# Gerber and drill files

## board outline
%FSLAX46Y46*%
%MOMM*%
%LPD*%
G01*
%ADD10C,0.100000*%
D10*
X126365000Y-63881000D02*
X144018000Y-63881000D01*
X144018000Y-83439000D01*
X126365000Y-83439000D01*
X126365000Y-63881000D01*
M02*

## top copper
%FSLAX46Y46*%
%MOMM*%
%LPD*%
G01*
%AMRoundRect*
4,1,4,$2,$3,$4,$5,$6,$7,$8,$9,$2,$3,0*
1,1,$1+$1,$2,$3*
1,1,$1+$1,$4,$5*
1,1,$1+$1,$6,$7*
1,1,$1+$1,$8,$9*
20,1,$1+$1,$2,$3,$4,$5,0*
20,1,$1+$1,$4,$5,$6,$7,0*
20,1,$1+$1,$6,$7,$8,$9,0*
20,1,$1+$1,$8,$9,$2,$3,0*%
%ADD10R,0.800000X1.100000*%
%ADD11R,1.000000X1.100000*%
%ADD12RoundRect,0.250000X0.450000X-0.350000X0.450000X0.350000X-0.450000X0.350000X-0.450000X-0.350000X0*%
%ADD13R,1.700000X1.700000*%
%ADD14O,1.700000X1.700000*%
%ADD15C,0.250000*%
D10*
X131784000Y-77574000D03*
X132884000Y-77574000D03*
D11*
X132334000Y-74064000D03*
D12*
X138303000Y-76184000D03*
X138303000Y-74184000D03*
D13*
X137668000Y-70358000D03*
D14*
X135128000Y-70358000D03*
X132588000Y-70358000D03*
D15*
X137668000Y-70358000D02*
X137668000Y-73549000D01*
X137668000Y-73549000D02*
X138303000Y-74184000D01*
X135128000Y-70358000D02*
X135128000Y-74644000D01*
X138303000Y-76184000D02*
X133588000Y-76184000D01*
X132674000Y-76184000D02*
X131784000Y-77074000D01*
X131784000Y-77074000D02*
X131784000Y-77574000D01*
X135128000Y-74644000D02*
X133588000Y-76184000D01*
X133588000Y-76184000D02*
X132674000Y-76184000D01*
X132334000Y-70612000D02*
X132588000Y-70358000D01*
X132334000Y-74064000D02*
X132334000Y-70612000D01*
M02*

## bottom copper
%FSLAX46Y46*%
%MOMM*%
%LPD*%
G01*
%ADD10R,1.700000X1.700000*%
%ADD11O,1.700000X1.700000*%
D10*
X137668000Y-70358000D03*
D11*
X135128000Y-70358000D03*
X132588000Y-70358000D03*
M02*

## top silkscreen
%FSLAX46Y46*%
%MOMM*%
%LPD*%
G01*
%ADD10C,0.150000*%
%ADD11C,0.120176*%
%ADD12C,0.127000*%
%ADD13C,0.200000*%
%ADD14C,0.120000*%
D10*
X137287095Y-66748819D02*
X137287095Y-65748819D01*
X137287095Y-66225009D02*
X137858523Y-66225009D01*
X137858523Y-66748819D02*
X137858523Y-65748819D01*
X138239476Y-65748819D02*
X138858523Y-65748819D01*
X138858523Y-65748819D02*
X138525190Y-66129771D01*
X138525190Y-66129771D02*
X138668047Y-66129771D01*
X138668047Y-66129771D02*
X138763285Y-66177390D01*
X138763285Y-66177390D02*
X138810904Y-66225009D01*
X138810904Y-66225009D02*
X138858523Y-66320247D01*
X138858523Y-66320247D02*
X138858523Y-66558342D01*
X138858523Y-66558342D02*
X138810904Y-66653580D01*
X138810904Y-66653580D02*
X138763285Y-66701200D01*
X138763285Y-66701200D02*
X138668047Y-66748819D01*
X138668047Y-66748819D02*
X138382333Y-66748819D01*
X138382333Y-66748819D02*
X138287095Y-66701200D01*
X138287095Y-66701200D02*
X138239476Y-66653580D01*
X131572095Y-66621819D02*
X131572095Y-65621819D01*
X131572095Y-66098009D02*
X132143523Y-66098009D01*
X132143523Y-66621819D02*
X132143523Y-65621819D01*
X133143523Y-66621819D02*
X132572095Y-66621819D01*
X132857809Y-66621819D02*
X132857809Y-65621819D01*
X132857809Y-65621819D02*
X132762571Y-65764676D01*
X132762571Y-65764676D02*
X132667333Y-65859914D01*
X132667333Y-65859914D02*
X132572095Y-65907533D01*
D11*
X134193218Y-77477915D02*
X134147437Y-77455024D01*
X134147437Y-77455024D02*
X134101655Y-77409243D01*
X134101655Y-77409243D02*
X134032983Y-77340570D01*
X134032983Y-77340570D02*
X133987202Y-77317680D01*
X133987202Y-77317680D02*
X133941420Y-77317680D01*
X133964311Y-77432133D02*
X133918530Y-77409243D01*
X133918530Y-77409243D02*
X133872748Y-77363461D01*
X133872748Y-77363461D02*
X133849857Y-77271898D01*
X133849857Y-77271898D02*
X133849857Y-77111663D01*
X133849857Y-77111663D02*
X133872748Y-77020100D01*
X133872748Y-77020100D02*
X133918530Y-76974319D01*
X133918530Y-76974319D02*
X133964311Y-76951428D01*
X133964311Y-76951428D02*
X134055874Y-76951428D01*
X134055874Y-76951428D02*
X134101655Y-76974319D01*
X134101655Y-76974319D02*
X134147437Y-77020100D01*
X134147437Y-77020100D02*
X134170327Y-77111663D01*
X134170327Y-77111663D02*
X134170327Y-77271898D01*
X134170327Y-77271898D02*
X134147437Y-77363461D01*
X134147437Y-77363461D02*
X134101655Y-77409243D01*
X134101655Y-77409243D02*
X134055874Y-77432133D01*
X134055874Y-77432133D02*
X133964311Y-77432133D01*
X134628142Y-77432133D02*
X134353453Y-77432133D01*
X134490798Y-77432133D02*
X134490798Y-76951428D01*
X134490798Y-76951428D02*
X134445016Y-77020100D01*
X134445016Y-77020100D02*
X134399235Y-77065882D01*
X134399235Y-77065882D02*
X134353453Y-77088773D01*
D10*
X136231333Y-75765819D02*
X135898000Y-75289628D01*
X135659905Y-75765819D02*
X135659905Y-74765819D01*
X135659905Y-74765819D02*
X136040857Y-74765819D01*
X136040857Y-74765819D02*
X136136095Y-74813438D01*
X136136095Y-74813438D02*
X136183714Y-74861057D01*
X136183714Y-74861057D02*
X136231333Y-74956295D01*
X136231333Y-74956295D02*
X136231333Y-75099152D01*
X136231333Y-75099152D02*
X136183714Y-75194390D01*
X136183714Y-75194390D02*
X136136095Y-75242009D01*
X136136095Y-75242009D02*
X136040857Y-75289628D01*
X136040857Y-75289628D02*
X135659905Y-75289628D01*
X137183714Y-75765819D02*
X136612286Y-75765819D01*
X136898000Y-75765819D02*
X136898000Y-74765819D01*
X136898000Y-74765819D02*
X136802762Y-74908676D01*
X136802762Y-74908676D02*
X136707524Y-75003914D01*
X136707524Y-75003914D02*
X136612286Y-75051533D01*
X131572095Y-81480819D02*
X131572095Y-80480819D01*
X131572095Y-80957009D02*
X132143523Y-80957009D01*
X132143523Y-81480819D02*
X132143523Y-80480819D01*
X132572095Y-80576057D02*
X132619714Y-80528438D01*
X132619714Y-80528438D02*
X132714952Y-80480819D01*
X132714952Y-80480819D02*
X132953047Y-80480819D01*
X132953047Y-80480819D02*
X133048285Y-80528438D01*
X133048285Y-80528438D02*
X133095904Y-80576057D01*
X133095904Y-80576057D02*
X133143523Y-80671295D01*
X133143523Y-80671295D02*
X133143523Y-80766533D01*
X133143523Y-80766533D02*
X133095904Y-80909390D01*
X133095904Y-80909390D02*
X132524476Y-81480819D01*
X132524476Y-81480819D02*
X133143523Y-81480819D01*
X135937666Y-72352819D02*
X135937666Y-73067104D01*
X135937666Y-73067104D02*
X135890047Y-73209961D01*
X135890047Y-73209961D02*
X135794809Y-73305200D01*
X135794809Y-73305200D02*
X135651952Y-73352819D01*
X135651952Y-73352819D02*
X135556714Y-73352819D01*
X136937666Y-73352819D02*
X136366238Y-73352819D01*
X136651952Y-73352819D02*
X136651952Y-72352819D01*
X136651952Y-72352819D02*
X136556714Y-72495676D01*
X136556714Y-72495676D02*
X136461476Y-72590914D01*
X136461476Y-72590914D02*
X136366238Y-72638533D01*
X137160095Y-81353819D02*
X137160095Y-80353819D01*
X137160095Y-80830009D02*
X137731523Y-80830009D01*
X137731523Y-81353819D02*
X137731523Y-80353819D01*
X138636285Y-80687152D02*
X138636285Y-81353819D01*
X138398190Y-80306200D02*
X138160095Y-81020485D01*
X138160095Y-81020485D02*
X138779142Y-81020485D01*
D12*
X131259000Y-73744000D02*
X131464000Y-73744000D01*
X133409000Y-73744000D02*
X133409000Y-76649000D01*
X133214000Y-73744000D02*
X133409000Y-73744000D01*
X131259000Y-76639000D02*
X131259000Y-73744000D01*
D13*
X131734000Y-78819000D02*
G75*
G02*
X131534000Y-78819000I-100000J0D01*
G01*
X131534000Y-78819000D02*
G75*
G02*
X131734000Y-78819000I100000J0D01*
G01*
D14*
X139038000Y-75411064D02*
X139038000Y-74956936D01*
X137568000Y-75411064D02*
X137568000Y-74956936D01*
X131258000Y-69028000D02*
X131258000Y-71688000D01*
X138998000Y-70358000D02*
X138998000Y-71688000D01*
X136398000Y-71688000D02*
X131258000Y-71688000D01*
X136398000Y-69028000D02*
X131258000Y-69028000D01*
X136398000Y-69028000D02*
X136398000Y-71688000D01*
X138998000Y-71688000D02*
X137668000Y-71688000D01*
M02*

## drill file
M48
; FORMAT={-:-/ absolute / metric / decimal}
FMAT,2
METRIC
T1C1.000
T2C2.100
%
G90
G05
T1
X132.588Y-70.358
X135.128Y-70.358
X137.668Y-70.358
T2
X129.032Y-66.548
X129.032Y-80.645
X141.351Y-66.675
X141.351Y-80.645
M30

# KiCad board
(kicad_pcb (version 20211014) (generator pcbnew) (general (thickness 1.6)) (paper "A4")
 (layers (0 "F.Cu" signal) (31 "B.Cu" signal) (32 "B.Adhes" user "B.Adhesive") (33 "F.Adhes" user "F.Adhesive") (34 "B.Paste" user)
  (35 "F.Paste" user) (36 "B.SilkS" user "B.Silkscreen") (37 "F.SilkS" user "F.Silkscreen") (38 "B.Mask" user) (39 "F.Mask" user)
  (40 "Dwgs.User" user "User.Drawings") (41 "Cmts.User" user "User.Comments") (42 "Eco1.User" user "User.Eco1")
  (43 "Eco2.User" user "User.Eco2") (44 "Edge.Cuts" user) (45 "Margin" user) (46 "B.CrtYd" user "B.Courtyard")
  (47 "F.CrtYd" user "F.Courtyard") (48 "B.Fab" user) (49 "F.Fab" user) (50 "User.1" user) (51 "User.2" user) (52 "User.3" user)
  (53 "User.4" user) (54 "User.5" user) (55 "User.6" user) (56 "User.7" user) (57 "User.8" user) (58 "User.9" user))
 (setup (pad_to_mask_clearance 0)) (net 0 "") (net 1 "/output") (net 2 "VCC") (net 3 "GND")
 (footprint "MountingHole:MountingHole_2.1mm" (layer "F.Cu") (at 141.351 66.675)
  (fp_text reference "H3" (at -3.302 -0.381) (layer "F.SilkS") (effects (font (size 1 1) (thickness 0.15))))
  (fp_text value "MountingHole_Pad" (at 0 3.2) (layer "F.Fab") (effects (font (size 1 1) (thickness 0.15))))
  (pad "" np_thru_hole circle (at 0 0) (size 2.1 2.1) (drill 2.1) (layers *.Cu *.Mask)))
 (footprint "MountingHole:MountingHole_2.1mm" (layer "F.Cu") (at 129.032 66.548)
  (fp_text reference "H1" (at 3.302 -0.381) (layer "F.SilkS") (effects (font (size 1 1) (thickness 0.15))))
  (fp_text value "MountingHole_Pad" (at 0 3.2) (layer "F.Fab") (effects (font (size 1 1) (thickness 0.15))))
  (pad "" np_thru_hole circle (at 0 0) (size 2.1 2.1) (drill 2.1) (layers *.Cu *.Mask)))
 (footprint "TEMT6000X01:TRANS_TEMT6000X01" (layer "F.Cu") (at 132.334 75.819 90)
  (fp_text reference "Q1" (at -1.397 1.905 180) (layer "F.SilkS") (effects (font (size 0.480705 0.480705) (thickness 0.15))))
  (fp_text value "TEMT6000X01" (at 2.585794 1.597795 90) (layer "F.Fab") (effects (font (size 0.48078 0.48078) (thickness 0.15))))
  (fp_line (start 2.075 -1.075) (end 2.075 -0.87) (layer "F.SilkS") (width 0.127))
  (fp_line (start 2.075 1.075) (end -0.83 1.075) (layer "F.SilkS") (width 0.127))
  (fp_line (start 2.075 0.88) (end 2.075 1.075) (layer "F.SilkS") (width 0.127))
  (fp_line (start -0.82 -1.075) (end 2.075 -1.075) (layer "F.SilkS") (width 0.127))
  (fp_circle (center -3 -0.7) (end -2.9 -0.7) (layer "F.SilkS") (width 0.2) (fill none))
  (pad "1" smd rect locked (at -1.755 -0.55 90) (size 1.1 0.8) (layers "F.Cu" "F.Paste" "F.Mask") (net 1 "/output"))
  (pad "2" smd rect locked (at -1.755 0.55 90) (size 1.1 0.8) (layers "F.Cu" "F.Paste" "F.Mask"))
  (pad "3" smd rect locked (at 1.755 0 90) (size 1.1 1) (layers "F.Cu" "F.Paste" "F.Mask") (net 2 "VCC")))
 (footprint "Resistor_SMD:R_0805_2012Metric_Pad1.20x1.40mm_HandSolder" (layer "F.Cu") (at 138.303 75.184 90)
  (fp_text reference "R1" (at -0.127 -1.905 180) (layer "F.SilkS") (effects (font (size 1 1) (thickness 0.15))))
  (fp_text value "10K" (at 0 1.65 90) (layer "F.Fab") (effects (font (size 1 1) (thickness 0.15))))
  (fp_line (start -0.227064 0.735) (end 0.227064 0.735) (layer "F.SilkS") (width 0.12))
  (fp_line (start -0.227064 -0.735) (end 0.227064 -0.735) (layer "F.SilkS") (width 0.12))
  (pad "1" smd roundrect (at -1 0 90) (size 1.2 1.4) (layers "F.Cu" "F.Paste" "F.Mask") (roundrect_rratio 0.208333) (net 1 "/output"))
  (pad "2" smd roundrect (at 1 0 90) (size 1.2 1.4) (layers "F.Cu" "F.Paste" "F.Mask") (roundrect_rratio 0.208333) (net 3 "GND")))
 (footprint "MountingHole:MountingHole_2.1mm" (layer "F.Cu") (at 129.032 80.645)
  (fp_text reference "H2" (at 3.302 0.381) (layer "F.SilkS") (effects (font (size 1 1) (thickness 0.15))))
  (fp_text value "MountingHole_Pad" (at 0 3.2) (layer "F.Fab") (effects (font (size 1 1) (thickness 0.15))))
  (pad "" np_thru_hole circle (at 0 0) (size 2.1 2.1) (drill 2.1) (layers *.Cu *.Mask)))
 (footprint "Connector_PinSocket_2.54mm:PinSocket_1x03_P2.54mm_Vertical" (layer "F.Cu") (at 137.668 70.358 -90)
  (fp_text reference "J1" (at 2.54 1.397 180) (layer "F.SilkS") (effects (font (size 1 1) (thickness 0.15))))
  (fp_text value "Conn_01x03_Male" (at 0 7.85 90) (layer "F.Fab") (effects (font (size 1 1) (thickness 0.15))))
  (fp_line (start -1.33 6.41) (end 1.33 6.41) (layer "F.SilkS") (width 0.12))
  (fp_line (start 0 -1.33) (end 1.33 -1.33) (layer "F.SilkS") (width 0.12))
  (fp_line (start 1.33 1.27) (end 1.33 6.41) (layer "F.SilkS") (width 0.12))
  (fp_line (start -1.33 1.27) (end -1.33 6.41) (layer "F.SilkS") (width 0.12))
  (fp_line (start -1.33 1.27) (end 1.33 1.27) (layer "F.SilkS") (width 0.12))
  (fp_line (start 1.33 -1.33) (end 1.33 0) (layer "F.SilkS") (width 0.12))
  (pad "1" thru_hole rect (at 0 0 270) (size 1.7 1.7) (drill 1) (layers *.Cu *.Mask) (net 3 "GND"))
  (pad "2" thru_hole oval (at 0 2.54 270) (size 1.7 1.7) (drill 1) (layers *.Cu *.Mask) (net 1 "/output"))
  (pad "3" thru_hole oval (at 0 5.08 270) (size 1.7 1.7) (drill 1) (layers *.Cu *.Mask) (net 2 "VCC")))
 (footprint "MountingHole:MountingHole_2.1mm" (layer "F.Cu") (at 141.351 80.645)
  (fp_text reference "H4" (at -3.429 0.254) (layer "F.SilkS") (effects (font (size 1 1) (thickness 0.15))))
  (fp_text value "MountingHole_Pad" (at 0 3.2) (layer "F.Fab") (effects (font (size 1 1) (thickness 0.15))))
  (pad "" np_thru_hole circle (at 0 0) (size 2.1 2.1) (drill 2.1) (layers *.Cu *.Mask)))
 (gr_rect (start 126.365 63.881) (end 144.018 83.439) (layer "Edge.Cuts") (width 0.1) (fill none))
 (segment (start 137.668 70.358) (end 137.668 73.549) (width 0.25) (layer "F.Cu") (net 3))
 (segment (start 137.668 73.549) (end 138.303 74.184) (width 0.25) (layer "F.Cu") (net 3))
 (segment (start 135.128 70.358) (end 135.128 74.644) (width 0.25) (layer "F.Cu") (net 1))
 (segment (start 138.303 76.184) (end 133.588 76.184) (width 0.25) (layer "F.Cu") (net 1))
 (segment (start 132.674 76.184) (end 131.784 77.074) (width 0.25) (layer "F.Cu") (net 1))
 (segment (start 131.784 77.074) (end 131.784 77.574) (width 0.25) (layer "F.Cu") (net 1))
 (segment (start 135.128 74.644) (end 133.588 76.184) (width 0.25) (layer "F.Cu") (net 1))
 (segment (start 133.588 76.184) (end 132.674 76.184) (width 0.25) (layer "F.Cu") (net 1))
 (segment (start 132.334 70.612) (end 132.588 70.358) (width 0.25) (layer "F.Cu") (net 2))
 (segment (start 132.334 74.064) (end 132.334 70.612) (width 0.25) (layer "F.Cu") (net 2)))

